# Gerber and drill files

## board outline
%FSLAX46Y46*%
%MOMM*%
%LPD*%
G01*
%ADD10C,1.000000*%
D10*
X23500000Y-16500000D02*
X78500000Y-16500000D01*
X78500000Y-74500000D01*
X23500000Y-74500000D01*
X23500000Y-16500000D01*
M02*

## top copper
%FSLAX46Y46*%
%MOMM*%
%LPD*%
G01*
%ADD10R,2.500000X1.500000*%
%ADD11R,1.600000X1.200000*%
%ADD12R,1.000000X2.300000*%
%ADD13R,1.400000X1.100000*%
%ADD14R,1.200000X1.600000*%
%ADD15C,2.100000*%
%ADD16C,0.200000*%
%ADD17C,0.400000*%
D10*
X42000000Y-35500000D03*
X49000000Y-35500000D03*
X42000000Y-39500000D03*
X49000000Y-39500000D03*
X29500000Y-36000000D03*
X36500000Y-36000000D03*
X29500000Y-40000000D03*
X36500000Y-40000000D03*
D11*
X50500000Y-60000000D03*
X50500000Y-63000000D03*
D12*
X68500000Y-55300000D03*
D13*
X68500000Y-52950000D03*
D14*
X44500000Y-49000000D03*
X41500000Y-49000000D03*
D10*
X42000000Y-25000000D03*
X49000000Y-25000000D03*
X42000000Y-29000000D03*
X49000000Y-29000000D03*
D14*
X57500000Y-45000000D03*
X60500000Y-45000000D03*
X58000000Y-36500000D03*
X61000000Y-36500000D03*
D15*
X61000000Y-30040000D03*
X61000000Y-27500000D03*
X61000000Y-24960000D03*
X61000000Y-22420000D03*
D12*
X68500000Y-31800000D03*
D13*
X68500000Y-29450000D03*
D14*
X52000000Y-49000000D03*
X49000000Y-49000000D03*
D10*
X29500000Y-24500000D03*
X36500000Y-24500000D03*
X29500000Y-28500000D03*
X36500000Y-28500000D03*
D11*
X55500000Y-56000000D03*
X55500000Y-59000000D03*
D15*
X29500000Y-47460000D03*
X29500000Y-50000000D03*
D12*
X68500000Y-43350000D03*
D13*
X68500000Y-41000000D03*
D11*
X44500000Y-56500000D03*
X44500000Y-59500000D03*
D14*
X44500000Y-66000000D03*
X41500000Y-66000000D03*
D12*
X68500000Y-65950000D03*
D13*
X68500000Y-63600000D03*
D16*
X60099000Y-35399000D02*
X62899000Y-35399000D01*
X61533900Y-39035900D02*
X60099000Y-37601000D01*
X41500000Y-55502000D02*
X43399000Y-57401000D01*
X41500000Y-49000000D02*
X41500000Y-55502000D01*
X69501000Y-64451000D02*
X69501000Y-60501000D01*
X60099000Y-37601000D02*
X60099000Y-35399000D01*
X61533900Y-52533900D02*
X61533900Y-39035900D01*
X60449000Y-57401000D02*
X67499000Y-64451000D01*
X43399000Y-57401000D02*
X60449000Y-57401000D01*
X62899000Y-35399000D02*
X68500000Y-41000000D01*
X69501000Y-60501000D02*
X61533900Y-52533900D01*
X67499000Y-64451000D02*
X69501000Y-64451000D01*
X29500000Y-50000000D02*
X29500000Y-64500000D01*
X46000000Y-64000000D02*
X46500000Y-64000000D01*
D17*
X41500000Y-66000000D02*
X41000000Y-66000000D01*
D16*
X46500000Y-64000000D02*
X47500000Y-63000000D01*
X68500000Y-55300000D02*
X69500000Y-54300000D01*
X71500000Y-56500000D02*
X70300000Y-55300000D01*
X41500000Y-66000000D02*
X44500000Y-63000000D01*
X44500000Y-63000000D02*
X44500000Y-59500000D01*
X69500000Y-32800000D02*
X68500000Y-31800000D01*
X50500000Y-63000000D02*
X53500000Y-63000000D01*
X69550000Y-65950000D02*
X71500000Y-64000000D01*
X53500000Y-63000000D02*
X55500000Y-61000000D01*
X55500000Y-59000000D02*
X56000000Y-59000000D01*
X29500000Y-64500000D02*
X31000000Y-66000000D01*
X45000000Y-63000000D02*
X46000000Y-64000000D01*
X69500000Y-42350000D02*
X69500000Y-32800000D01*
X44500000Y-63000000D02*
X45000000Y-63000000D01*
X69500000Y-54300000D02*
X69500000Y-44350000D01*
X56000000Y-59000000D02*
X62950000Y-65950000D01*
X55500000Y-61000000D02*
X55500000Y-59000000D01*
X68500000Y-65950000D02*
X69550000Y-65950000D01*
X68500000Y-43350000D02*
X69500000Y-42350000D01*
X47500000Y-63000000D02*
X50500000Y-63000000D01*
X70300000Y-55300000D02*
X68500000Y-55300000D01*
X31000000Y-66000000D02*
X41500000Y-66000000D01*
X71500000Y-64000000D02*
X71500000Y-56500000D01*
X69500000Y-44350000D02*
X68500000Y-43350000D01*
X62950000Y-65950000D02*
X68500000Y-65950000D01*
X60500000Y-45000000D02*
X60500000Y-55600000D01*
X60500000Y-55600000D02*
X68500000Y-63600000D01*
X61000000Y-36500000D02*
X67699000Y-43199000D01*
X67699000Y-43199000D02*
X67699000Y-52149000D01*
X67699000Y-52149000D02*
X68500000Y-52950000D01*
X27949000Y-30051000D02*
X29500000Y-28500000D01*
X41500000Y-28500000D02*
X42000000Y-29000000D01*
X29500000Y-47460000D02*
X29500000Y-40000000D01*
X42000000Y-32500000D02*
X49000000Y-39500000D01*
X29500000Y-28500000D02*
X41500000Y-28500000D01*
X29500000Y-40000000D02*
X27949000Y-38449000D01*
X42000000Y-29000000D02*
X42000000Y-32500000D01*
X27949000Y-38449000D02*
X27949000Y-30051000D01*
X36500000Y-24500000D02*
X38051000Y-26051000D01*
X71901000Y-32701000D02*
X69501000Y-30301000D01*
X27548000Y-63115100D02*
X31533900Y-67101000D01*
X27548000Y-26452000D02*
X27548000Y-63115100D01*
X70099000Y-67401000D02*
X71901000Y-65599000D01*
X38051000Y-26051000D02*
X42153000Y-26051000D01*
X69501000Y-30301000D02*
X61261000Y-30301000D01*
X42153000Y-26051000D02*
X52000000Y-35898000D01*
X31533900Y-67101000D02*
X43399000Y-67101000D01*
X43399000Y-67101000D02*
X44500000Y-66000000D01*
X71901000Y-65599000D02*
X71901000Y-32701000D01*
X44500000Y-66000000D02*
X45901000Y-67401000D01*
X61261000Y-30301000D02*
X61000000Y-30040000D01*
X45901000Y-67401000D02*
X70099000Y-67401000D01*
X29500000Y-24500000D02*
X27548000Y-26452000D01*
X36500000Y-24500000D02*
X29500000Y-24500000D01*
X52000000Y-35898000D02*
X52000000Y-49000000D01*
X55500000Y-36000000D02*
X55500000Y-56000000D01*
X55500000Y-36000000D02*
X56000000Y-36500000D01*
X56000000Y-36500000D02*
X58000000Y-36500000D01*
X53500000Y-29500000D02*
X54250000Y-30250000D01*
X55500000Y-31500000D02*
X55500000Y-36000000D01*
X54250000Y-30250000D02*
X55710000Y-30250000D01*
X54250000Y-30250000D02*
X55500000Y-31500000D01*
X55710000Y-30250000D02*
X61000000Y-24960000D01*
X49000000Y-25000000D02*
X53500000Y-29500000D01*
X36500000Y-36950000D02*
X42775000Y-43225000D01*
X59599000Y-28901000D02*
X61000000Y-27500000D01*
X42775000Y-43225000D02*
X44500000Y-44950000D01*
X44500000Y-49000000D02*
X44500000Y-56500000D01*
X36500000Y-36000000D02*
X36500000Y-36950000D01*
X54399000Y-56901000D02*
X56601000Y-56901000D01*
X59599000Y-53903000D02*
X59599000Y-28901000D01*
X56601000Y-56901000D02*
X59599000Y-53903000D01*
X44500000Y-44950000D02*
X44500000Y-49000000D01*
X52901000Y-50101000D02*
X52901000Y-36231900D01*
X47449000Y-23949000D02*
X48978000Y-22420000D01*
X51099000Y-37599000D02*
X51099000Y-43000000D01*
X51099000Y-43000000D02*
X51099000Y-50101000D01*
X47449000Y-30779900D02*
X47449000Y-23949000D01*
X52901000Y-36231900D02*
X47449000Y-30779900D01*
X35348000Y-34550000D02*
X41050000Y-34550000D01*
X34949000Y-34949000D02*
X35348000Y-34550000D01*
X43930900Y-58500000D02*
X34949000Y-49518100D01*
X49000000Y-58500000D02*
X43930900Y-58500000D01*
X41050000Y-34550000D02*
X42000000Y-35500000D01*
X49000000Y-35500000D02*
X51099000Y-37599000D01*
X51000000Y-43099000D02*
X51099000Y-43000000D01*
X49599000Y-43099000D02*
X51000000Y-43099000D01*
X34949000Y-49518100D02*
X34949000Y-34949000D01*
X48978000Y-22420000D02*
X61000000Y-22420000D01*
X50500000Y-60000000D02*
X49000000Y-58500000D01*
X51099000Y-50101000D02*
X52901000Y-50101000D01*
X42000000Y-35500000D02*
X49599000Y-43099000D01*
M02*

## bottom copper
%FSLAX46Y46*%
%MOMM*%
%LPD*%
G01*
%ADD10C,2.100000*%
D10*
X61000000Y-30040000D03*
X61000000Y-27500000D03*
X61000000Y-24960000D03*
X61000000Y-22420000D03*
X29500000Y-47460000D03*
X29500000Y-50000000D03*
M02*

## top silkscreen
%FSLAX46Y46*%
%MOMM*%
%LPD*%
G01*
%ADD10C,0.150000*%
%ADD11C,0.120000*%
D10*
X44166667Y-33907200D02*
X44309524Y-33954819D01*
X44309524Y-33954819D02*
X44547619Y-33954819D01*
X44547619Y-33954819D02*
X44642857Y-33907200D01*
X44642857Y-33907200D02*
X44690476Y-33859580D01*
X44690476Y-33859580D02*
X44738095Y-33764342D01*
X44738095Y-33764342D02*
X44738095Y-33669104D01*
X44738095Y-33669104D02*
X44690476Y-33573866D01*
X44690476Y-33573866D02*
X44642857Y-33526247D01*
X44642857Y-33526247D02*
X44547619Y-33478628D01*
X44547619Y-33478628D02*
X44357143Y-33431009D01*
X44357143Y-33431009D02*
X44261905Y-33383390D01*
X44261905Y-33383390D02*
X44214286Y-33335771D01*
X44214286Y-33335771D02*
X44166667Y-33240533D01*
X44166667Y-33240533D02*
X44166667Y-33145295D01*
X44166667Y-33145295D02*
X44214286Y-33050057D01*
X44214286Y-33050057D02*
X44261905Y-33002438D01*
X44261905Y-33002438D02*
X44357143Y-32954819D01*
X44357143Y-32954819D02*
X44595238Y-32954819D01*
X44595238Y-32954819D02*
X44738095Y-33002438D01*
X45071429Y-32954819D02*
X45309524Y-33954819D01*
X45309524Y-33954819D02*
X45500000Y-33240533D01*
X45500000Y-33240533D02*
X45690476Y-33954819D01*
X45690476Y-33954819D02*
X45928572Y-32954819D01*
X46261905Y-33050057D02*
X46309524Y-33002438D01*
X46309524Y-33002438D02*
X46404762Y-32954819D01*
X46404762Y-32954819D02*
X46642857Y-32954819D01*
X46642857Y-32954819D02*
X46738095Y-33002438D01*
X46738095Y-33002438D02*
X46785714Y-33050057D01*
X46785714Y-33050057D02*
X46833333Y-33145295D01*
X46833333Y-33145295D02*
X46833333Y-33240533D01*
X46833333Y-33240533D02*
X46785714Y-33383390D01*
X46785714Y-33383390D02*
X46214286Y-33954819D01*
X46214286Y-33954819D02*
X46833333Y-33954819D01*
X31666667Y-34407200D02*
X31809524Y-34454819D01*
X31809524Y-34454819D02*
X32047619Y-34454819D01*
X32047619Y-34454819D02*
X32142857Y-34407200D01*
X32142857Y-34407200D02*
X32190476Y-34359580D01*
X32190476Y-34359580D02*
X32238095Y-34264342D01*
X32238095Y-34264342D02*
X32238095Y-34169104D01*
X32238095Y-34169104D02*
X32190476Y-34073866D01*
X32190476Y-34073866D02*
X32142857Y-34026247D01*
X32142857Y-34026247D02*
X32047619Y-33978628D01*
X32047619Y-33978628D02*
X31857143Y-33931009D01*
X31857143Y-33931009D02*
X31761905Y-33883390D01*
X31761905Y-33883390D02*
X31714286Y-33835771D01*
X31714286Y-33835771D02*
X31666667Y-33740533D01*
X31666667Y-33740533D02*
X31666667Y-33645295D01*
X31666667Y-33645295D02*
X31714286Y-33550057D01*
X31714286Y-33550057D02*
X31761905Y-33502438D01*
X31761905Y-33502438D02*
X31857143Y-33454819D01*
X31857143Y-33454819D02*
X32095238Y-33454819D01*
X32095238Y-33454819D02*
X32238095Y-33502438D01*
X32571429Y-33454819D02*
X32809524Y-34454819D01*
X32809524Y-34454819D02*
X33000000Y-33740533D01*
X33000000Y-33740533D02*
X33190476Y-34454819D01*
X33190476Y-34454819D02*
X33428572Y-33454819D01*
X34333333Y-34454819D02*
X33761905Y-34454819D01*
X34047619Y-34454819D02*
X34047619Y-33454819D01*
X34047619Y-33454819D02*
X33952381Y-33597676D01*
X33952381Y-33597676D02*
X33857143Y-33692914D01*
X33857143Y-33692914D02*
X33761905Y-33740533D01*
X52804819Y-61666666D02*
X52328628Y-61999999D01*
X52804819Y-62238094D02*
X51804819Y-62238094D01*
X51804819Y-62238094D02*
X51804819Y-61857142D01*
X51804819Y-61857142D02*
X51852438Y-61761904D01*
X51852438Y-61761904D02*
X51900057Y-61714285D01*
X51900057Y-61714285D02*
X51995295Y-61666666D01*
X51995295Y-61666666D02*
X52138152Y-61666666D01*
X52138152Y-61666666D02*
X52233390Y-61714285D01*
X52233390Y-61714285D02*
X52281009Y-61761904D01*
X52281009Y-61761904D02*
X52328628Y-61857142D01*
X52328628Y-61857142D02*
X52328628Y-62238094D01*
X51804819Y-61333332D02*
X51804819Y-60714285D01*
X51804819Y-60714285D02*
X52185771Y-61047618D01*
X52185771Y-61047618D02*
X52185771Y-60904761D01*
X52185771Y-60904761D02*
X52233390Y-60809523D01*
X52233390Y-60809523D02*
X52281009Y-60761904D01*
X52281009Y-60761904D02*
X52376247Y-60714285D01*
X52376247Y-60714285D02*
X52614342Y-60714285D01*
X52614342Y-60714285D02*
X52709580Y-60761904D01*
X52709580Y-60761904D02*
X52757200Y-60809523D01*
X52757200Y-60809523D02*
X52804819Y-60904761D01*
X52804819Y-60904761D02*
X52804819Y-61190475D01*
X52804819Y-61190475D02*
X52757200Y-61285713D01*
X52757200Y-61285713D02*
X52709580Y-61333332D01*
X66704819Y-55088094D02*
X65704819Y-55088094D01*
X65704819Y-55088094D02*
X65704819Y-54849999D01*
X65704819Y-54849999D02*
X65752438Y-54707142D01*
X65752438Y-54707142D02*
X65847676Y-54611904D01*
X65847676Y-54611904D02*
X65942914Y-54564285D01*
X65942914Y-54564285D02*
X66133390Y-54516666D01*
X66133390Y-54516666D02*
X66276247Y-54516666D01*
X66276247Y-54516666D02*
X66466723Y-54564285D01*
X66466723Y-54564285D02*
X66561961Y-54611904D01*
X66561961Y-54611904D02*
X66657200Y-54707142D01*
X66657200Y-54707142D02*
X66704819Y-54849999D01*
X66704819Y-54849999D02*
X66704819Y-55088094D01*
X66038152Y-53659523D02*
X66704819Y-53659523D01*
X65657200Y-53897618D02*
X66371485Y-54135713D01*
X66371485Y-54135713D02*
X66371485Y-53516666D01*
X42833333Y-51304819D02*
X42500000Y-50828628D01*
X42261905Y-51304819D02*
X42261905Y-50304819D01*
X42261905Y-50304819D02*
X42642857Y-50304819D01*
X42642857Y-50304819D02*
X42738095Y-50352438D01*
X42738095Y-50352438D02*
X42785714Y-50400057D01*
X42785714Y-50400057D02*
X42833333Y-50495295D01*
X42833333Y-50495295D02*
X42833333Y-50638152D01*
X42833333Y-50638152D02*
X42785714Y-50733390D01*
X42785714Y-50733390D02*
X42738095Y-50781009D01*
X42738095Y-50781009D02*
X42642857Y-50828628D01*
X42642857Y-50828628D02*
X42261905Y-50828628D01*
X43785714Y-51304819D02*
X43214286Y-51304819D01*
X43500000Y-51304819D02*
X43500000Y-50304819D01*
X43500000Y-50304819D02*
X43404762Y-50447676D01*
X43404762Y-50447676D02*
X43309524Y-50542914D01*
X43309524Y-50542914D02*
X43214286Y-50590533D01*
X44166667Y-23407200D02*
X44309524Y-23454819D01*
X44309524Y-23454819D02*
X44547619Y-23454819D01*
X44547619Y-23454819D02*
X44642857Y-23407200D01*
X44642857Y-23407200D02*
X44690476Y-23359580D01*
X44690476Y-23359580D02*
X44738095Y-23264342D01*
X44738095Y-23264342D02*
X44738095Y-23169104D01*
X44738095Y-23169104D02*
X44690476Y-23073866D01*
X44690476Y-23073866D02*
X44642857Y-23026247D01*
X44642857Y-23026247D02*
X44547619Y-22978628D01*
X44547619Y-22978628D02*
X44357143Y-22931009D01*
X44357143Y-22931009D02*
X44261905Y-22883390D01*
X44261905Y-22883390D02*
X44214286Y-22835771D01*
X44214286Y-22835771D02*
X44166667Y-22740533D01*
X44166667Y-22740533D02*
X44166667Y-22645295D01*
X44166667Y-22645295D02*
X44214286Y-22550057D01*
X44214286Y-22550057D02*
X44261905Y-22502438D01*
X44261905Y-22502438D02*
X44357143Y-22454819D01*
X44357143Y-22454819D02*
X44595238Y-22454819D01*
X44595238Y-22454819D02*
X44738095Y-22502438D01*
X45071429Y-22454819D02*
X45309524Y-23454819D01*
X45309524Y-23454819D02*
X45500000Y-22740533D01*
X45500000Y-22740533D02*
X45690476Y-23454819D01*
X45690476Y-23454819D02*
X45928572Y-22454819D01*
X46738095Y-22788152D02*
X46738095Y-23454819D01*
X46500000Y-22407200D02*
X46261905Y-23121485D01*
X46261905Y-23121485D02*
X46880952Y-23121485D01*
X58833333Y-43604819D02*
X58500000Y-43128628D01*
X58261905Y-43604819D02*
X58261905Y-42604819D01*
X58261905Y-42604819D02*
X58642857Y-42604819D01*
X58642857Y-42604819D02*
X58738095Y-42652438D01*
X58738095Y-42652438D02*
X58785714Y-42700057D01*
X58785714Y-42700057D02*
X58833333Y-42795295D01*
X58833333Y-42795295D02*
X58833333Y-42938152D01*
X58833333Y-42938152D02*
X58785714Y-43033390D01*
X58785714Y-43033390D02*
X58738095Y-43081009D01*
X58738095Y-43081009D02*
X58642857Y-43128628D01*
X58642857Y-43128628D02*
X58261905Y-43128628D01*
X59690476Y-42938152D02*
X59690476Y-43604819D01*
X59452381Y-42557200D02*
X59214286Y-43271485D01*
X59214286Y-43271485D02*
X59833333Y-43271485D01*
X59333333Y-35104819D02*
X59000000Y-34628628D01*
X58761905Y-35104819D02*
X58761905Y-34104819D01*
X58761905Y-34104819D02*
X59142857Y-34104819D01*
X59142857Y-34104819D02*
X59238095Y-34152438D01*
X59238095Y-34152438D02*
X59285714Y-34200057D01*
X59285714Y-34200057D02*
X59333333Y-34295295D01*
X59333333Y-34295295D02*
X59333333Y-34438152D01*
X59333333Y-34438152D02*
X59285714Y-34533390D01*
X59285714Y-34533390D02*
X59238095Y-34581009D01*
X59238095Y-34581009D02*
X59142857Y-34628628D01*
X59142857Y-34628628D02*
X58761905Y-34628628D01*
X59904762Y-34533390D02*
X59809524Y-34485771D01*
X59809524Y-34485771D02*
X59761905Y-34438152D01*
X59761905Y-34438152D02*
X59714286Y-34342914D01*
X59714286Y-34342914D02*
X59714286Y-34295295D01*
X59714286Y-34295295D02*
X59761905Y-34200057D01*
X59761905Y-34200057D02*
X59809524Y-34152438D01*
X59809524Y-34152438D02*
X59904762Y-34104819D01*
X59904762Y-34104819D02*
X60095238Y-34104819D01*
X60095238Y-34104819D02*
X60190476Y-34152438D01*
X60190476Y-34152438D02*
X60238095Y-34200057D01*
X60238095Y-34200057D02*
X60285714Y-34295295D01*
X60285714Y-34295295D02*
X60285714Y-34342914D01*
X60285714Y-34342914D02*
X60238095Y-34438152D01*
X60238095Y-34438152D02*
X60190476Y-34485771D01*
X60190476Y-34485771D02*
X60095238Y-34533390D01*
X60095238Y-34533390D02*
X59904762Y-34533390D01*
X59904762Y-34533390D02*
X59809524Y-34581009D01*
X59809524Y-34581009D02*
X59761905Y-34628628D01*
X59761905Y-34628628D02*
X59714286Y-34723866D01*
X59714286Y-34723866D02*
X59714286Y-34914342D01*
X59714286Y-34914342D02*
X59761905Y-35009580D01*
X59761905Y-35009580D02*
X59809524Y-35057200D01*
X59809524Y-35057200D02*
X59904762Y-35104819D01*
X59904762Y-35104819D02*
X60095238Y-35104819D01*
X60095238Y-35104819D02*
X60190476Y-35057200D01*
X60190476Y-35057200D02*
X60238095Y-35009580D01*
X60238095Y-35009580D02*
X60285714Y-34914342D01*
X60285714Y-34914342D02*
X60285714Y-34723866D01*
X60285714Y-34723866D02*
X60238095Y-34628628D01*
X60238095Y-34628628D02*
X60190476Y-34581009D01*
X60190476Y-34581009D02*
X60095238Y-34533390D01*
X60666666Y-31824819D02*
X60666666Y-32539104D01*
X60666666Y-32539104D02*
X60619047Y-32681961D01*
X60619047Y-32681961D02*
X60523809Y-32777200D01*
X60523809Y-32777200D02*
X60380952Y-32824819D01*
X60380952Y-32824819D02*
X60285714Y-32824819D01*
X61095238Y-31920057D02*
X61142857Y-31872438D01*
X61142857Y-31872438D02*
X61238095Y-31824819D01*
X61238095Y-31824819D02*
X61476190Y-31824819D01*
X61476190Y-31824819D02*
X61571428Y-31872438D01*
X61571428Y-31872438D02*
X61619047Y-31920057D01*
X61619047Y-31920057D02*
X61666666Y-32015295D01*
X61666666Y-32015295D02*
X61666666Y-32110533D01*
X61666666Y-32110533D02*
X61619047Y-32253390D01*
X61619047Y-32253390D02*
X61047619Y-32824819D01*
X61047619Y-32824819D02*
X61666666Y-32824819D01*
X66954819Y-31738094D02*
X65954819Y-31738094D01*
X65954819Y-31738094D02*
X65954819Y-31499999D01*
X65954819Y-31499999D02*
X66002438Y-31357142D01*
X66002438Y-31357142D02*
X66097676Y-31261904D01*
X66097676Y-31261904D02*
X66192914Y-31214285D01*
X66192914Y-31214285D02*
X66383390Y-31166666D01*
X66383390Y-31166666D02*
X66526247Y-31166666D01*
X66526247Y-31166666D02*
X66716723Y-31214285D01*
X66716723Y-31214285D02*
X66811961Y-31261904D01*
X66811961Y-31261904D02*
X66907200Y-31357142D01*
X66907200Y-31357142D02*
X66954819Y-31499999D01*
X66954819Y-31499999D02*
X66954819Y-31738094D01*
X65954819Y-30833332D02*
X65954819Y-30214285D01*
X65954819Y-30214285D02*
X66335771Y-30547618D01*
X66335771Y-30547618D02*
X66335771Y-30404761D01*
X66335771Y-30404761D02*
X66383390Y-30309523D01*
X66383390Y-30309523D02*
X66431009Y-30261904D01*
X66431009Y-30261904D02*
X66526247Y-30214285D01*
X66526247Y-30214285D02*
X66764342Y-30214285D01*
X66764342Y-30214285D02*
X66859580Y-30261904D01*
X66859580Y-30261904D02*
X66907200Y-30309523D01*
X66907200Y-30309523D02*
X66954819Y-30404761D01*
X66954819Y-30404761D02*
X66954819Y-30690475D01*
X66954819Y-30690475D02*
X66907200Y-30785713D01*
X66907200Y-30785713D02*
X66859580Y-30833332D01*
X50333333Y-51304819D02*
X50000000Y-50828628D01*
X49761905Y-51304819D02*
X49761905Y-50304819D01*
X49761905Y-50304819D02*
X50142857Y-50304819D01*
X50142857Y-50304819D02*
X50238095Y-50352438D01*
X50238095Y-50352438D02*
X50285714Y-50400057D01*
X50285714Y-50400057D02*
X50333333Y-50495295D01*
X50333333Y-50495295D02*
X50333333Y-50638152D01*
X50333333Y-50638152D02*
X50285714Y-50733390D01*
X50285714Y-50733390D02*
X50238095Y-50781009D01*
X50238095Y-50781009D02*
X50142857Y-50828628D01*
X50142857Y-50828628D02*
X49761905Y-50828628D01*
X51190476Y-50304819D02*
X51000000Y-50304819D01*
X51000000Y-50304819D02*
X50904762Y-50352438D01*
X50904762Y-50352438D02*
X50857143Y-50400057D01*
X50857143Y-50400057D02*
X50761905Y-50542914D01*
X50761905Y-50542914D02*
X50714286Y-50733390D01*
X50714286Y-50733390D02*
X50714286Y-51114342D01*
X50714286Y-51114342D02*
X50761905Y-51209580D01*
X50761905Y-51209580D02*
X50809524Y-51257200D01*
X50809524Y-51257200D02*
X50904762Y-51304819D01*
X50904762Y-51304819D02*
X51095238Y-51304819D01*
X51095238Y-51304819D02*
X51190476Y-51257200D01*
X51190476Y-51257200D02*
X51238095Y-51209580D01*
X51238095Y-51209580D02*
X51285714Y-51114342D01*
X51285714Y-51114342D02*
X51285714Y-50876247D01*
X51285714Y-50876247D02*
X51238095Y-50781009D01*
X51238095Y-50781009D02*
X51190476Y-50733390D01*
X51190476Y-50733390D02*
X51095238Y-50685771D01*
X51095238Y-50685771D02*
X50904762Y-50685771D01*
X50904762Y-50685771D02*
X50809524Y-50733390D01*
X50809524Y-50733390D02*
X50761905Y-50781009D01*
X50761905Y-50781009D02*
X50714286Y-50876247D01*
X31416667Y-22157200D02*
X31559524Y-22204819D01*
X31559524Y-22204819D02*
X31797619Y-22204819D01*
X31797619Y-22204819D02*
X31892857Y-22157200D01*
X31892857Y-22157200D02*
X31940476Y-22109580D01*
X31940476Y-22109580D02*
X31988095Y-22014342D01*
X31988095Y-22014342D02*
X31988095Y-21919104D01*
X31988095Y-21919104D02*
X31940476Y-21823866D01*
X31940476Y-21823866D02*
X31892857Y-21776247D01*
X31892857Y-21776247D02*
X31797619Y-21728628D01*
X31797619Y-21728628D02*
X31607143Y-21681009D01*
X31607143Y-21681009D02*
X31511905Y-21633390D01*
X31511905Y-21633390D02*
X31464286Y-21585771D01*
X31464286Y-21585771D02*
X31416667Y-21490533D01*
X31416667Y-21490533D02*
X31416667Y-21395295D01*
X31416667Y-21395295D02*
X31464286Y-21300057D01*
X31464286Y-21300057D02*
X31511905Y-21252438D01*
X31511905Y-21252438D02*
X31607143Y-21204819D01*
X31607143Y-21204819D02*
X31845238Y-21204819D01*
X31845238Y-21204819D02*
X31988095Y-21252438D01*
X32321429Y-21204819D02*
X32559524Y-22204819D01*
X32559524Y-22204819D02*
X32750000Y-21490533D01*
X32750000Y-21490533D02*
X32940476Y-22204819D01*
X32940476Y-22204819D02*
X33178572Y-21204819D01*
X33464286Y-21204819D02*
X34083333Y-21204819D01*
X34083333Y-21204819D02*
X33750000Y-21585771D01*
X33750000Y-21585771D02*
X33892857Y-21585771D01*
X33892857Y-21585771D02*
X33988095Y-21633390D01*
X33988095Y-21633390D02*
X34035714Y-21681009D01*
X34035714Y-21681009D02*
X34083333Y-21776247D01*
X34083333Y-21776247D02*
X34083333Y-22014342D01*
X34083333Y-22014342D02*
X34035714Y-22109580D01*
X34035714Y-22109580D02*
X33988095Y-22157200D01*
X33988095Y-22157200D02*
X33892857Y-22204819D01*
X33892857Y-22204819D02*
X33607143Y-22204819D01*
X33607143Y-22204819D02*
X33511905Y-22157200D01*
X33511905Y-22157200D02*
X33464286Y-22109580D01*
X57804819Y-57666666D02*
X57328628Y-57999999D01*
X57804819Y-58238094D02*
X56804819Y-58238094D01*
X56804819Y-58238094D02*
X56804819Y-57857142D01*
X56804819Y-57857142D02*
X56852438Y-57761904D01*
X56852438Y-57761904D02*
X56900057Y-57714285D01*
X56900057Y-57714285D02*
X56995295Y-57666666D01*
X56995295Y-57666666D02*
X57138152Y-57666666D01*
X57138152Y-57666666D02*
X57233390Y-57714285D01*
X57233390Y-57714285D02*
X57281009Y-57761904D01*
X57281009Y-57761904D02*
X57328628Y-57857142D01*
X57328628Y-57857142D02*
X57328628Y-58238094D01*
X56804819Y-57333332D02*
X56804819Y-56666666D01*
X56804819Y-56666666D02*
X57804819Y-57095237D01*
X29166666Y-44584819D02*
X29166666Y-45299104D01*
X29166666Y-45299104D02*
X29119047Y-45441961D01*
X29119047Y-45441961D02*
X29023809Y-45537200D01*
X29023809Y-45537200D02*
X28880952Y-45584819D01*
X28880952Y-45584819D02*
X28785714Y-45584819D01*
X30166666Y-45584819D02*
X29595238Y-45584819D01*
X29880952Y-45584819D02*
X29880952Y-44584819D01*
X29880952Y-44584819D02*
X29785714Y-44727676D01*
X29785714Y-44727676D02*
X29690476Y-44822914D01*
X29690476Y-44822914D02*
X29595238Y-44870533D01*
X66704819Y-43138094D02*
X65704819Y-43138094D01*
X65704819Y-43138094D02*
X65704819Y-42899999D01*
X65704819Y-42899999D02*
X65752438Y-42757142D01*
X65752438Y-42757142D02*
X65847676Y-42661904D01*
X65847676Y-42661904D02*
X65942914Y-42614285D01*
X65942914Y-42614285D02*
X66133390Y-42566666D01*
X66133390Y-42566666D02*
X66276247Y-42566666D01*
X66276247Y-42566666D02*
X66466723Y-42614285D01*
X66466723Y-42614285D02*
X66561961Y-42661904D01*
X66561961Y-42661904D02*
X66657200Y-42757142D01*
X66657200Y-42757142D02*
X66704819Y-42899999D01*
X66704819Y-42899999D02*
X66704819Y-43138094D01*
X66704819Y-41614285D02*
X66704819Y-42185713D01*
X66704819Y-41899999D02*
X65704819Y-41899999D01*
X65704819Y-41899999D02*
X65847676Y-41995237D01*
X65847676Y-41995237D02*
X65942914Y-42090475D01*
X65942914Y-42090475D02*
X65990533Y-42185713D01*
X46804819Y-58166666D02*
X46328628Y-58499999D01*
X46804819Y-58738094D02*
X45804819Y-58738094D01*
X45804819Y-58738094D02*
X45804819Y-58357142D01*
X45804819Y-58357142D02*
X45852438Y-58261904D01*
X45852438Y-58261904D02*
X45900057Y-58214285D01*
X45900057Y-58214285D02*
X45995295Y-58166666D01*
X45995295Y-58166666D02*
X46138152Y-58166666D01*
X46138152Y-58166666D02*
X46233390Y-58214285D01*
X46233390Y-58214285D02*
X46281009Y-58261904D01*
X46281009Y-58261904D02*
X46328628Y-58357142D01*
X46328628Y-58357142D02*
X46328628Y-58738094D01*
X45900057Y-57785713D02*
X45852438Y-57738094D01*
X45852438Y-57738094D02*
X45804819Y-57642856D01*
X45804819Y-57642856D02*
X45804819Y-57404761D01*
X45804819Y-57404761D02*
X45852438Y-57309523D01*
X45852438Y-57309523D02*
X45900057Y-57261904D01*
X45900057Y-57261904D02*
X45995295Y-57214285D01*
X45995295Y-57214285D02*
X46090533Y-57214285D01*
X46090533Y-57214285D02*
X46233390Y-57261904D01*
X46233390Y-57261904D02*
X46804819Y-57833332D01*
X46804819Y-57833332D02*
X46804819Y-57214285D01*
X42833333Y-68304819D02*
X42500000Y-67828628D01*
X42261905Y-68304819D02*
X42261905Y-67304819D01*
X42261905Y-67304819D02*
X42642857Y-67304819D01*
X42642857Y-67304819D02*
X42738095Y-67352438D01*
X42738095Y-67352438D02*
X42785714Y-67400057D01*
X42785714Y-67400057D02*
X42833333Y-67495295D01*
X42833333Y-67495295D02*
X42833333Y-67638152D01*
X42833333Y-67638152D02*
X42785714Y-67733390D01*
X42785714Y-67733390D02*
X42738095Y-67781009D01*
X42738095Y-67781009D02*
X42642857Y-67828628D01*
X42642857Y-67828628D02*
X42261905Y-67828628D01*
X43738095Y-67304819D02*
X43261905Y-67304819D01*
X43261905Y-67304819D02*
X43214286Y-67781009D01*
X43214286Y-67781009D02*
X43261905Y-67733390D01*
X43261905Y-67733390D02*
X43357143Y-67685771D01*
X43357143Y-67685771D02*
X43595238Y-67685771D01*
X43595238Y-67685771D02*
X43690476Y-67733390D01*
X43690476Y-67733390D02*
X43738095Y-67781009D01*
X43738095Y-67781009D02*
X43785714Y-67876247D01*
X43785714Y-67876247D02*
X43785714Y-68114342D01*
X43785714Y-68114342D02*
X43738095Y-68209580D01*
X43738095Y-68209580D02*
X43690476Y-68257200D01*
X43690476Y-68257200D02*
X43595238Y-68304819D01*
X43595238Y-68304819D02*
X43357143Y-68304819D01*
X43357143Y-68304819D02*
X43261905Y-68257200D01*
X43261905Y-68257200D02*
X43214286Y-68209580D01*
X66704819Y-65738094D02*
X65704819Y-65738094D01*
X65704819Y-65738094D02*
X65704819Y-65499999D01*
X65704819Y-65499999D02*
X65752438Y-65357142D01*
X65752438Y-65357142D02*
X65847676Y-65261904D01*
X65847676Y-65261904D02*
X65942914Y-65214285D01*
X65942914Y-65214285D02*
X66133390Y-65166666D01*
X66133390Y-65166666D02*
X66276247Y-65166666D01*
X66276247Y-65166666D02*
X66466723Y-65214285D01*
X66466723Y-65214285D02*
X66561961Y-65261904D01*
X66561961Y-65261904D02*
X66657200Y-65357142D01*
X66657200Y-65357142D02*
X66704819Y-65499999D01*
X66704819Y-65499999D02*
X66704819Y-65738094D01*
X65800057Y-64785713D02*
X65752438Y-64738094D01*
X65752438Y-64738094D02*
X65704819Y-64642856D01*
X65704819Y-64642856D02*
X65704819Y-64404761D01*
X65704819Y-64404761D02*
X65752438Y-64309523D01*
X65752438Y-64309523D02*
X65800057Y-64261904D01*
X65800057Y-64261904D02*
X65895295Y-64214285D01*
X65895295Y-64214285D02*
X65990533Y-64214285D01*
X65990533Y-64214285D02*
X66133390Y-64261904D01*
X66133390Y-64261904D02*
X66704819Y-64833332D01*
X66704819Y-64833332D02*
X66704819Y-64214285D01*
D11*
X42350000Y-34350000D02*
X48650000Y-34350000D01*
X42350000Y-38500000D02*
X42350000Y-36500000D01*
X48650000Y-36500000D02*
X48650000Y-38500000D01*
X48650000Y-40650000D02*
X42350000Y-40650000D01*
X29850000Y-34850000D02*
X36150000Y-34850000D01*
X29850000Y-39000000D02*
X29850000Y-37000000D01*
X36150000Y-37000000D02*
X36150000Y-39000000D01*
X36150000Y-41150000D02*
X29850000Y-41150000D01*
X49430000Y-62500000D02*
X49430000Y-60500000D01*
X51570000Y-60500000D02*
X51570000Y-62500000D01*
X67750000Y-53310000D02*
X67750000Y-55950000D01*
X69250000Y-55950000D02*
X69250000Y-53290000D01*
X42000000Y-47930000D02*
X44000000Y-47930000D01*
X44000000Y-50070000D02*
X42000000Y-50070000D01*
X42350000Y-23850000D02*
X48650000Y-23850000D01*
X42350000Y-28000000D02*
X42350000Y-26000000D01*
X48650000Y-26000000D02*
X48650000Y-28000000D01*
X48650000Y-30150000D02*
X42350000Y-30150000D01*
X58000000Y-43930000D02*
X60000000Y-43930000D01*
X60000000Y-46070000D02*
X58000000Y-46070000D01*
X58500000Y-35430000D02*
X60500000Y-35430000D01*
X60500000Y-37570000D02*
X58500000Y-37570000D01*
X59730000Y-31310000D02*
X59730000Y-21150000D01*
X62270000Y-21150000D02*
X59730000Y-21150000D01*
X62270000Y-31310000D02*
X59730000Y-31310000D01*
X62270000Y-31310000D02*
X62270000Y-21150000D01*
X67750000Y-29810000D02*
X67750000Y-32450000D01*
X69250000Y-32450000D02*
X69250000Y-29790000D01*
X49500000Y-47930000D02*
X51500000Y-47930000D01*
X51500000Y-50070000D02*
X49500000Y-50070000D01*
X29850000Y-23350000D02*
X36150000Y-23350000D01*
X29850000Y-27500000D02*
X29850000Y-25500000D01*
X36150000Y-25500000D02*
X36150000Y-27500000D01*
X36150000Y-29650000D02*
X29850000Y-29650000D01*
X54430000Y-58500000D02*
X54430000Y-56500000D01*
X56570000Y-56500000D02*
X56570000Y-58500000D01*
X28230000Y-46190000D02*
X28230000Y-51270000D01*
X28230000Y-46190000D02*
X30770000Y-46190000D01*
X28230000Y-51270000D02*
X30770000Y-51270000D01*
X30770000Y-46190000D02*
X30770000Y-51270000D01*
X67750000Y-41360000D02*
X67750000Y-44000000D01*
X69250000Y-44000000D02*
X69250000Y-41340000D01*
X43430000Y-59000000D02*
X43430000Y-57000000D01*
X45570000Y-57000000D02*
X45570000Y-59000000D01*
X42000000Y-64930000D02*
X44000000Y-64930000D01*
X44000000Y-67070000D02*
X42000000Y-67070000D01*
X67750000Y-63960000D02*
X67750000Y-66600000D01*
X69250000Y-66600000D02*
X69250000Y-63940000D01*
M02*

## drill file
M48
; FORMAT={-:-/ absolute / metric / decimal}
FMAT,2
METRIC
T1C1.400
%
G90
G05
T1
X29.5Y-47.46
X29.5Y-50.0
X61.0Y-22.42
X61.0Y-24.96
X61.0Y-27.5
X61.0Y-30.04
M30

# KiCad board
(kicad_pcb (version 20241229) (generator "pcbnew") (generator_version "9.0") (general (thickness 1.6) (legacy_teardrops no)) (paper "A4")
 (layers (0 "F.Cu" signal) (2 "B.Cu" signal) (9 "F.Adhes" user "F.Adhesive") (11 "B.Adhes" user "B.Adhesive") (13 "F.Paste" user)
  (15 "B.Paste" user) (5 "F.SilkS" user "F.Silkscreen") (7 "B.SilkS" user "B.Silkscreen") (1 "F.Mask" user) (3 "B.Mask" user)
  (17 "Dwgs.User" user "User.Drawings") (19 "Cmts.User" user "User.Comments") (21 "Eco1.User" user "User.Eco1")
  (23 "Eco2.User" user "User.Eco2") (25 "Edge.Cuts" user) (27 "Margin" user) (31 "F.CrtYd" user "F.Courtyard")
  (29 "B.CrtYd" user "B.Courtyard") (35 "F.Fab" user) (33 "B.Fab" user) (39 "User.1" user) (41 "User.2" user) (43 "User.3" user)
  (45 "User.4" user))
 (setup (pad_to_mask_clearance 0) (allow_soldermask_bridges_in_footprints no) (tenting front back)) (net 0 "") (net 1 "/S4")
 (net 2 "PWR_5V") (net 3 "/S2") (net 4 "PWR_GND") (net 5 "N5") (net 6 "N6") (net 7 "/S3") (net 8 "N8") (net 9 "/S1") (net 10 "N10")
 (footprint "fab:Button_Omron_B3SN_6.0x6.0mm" (layer "F.Cu") (at 45.5 37.5)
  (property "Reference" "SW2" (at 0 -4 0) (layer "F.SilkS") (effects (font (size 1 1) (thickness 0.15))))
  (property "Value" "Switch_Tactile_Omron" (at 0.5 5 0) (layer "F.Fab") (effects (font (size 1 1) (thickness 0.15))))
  (fp_line (start -3.15 -3.15) (end 3.15 -3.15) (stroke (width 0.12) (type solid)) (layer "F.SilkS"))
  (fp_line (start -3.15 1) (end -3.15 -1) (stroke (width 0.12) (type solid)) (layer "F.SilkS"))
  (fp_line (start 3.15 -1) (end 3.15 1) (stroke (width 0.12) (type solid)) (layer "F.SilkS"))
  (fp_line (start 3.15 3.15) (end -3.15 3.15) (stroke (width 0.12) (type solid)) (layer "F.SilkS"))
  (pad "1" smd rect (at -3.5 -2) (size 2.5 1.5) (layers "F.Cu" "F.Mask" "F.Paste") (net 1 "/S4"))
  (pad "1" smd rect (at 3.5 -2) (size 2.5 1.5) (layers "F.Cu" "F.Mask" "F.Paste") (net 1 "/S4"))
  (pad "2" smd rect (at -3.5 2) (size 2.5 1.5) (layers "F.Cu" "F.Mask" "F.Paste") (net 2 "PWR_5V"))
  (pad "2" smd rect (at 3.5 2) (size 2.5 1.5) (layers "F.Cu" "F.Mask" "F.Paste") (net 2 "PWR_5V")))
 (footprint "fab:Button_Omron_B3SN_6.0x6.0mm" (layer "F.Cu") (at 33 38)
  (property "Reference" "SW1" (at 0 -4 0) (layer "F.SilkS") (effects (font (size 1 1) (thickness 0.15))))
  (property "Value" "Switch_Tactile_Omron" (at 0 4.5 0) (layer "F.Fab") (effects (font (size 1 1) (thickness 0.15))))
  (fp_line (start -3.15 -3.15) (end 3.15 -3.15) (stroke (width 0.12) (type solid)) (layer "F.SilkS"))
  (fp_line (start -3.15 1) (end -3.15 -1) (stroke (width 0.12) (type solid)) (layer "F.SilkS"))
  (fp_line (start 3.15 -1) (end 3.15 1) (stroke (width 0.12) (type solid)) (layer "F.SilkS"))
  (fp_line (start 3.15 3.15) (end -3.15 3.15) (stroke (width 0.12) (type solid)) (layer "F.SilkS"))
  (pad "1" smd rect (at -3.5 -2) (size 2.5 1.5) (layers "F.Cu" "F.Mask" "F.Paste") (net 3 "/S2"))
  (pad "1" smd rect (at 3.5 -2) (size 2.5 1.5) (layers "F.Cu" "F.Mask" "F.Paste") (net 3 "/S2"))
  (pad "2" smd rect (at -3.5 2) (size 2.5 1.5) (layers "F.Cu" "F.Mask" "F.Paste") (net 2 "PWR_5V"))
  (pad "2" smd rect (at 3.5 2) (size 2.5 1.5) (layers "F.Cu" "F.Mask" "F.Paste") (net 2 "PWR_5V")))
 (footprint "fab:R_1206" (layer "F.Cu") (at 50.5 61.5 -90)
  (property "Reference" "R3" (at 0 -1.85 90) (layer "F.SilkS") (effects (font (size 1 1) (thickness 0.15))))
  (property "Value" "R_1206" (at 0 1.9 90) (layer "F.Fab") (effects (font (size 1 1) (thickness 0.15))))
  (fp_line (start 1 1.07) (end -1 1.07) (stroke (width 0.12) (type solid)) (layer "F.SilkS"))
  (fp_line (start -1 -1.07) (end 1 -1.07) (stroke (width 0.12) (type solid)) (layer "F.SilkS"))
  (pad "1" smd rect (at -1.5 0 270) (size 1.2 1.6) (layers "F.Cu" "F.Mask" "F.Paste") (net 1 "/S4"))
  (pad "2" smd rect (at 1.5 0 270) (size 1.2 1.6) (layers "F.Cu" "F.Mask" "F.Paste") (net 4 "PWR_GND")))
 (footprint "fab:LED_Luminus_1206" (layer "F.Cu") (at 68.5 54.35 -90)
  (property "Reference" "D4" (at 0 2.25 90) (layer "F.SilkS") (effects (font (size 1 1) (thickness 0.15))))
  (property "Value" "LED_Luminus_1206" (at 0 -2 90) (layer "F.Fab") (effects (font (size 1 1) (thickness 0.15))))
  (fp_line (start -1.04 0.75) (end 1.6 0.75) (stroke (width 0.12) (type solid)) (layer "F.SilkS"))
  (fp_line (start 1.6 -0.75) (end -1.06 -0.75) (stroke (width 0.12) (type solid)) (layer "F.SilkS"))
  (pad "1" smd rect (at 0.95 0 270) (size 2.3 1) (layers "F.Cu" "F.Mask" "F.Paste") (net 4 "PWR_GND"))
  (pad "2" smd rect (at -1.4 0 270) (size 1.1 1.4) (layers "F.Cu" "F.Mask" "F.Paste") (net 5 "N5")))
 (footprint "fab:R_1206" (layer "F.Cu") (at 43 49 180)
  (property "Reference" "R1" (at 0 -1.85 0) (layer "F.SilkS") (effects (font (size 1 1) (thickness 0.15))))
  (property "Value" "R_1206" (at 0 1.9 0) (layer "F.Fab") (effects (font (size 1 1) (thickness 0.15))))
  (fp_line (start 1 1.07) (end -1 1.07) (stroke (width 0.12) (type solid)) (layer "F.SilkS"))
  (fp_line (start -1 -1.07) (end 1 -1.07) (stroke (width 0.12) (type solid)) (layer "F.SilkS"))
  (pad "1" smd rect (at -1.5 0 180) (size 1.2 1.6) (layers "F.Cu" "F.Mask" "F.Paste") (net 3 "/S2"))
  (pad "2" smd rect (at 1.5 0 180) (size 1.2 1.6) (layers "F.Cu" "F.Mask" "F.Paste") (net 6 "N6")))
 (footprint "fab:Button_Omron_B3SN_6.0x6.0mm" (layer "F.Cu") (at 45.5 27)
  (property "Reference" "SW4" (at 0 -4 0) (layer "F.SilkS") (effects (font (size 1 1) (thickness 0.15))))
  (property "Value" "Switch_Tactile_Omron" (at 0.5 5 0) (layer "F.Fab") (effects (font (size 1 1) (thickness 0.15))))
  (fp_line (start -3.15 -3.15) (end 3.15 -3.15) (stroke (width 0.12) (type solid)) (layer "F.SilkS"))
  (fp_line (start -3.15 1) (end -3.15 -1) (stroke (width 0.12) (type solid)) (layer "F.SilkS"))
  (fp_line (start 3.15 -1) (end 3.15 1) (stroke (width 0.12) (type solid)) (layer "F.SilkS"))
  (fp_line (start 3.15 3.15) (end -3.15 3.15) (stroke (width 0.12) (type solid)) (layer "F.SilkS"))
  (pad "1" smd rect (at -3.5 -2) (size 2.5 1.5) (layers "F.Cu" "F.Mask" "F.Paste") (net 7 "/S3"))
  (pad "1" smd rect (at 3.5 -2) (size 2.5 1.5) (layers "F.Cu" "F.Mask" "F.Paste") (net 7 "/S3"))
  (pad "2" smd rect (at -3.5 2) (size 2.5 1.5) (layers "F.Cu" "F.Mask" "F.Paste") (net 2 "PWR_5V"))
  (pad "2" smd rect (at 3.5 2) (size 2.5 1.5) (layers "F.Cu" "F.Mask" "F.Paste") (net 2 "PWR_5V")))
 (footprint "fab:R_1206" (layer "F.Cu") (at 59 45)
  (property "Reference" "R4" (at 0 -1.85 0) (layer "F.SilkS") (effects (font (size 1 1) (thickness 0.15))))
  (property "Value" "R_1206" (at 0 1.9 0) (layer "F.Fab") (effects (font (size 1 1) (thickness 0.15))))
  (fp_line (start -1 -1.07) (end 1 -1.07) (stroke (width 0.12) (type solid)) (layer "F.SilkS"))
  (fp_line (start 1 1.07) (end -1 1.07) (stroke (width 0.12) (type solid)) (layer "F.SilkS"))
  (pad "1" smd rect (at -1.5 0) (size 1.2 1.6) (layers "F.Cu" "F.Mask" "F.Paste") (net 1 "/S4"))
  (pad "2" smd rect (at 1.5 0) (size 1.2 1.6) (layers "F.Cu" "F.Mask" "F.Paste") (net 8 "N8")))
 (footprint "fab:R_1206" (layer "F.Cu") (at 59.5 36.5)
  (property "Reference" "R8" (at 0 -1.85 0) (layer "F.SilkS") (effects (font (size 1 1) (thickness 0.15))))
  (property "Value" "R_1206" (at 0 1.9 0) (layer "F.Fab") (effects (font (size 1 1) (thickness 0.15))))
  (fp_line (start -1 -1.07) (end 1 -1.07) (stroke (width 0.12) (type solid)) (layer "F.SilkS"))
  (fp_line (start 1 1.07) (end -1 1.07) (stroke (width 0.12) (type solid)) (layer "F.SilkS"))
  (pad "1" smd rect (at -1.5 0) (size 1.2 1.6) (layers "F.Cu" "F.Mask" "F.Paste") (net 7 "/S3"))
  (pad "2" smd rect (at 1.5 0) (size 1.2 1.6) (layers "F.Cu" "F.Mask" "F.Paste") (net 5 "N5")))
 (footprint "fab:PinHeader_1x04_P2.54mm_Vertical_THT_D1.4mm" (layer "F.Cu") (at 61 30.04 180)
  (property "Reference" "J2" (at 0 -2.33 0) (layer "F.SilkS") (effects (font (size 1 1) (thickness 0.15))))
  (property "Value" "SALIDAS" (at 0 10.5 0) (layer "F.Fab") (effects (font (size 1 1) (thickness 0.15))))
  (fp_line (start 1.27 -1.27) (end 1.27 8.89) (stroke (width 0.12) (type solid)) (layer "F.SilkS"))
  (fp_line (start -1.27 8.89) (end 1.27 8.89) (stroke (width 0.12) (type solid)) (layer "F.SilkS"))
  (fp_line (start -1.27 -1.27) (end 1.27 -1.27) (stroke (width 0.12) (type solid)) (layer "F.SilkS"))
  (fp_line (start -1.27 -1.27) (end -1.27 8.89) (stroke (width 0.12) (type solid)) (layer "F.SilkS"))
  (pad "1" thru_hole circle (at 0 0 180) (size 2.1 2.1) (drill 1.4) (layers "*.Cu" "*.Mask") (remove_unused_layers no) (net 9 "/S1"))
  (pad "2" thru_hole circle (at 0 2.54 180) (size 2.1 2.1) (drill 1.4) (layers "*.Cu" "*.Mask") (remove_unused_layers no) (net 3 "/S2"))
  (pad "3" thru_hole circle (at 0 5.08 180) (size 2.1 2.1) (drill 1.4) (layers "*.Cu" "*.Mask") (remove_unused_layers no) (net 7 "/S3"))
  (pad "4" thru_hole circle (at 0 7.62 180) (size 2.1 2.1) (drill 1.4) (layers "*.Cu" "*.Mask") (remove_unused_layers no) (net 1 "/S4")))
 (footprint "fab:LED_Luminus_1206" (layer "F.Cu") (at 68.5 30.85 -90)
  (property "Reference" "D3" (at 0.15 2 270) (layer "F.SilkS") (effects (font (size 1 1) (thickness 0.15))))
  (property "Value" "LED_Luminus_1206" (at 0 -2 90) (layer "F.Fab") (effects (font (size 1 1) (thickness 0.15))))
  (fp_line (start -1.04 0.75) (end 1.6 0.75) (stroke (width 0.12) (type solid)) (layer "F.SilkS"))
  (fp_line (start 1.6 -0.75) (end -1.06 -0.75) (stroke (width 0.12) (type solid)) (layer "F.SilkS"))
  (pad "1" smd rect (at 0.95 0 270) (size 2.3 1) (layers "F.Cu" "F.Mask" "F.Paste") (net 4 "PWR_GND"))
  (pad "2" smd rect (at -1.4 0 270) (size 1.1 1.4) (layers "F.Cu" "F.Mask" "F.Paste") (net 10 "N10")))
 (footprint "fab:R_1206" (layer "F.Cu") (at 50.5 49 180)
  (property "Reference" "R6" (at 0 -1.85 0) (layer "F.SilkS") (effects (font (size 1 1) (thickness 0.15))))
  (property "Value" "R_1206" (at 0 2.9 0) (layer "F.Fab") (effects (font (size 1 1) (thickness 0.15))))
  (fp_line (start 1 1.07) (end -1 1.07) (stroke (width 0.12) (type solid)) (layer "F.SilkS"))
  (fp_line (start -1 -1.07) (end 1 -1.07) (stroke (width 0.12) (type solid)) (layer "F.SilkS"))
  (pad "1" smd rect (at -1.5 0 180) (size 1.2 1.6) (layers "F.Cu" "F.Mask" "F.Paste") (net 9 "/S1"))
  (pad "2" smd rect (at 1.5 0 180) (size 1.2 1.6) (layers "F.Cu" "F.Mask" "F.Paste") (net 10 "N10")))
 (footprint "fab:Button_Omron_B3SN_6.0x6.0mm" (layer "F.Cu") (at 33 26.5)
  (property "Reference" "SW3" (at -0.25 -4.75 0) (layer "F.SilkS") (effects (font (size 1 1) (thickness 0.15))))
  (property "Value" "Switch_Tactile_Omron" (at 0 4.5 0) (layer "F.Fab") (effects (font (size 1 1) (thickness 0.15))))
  (fp_line (start -3.15 -3.15) (end 3.15 -3.15) (stroke (width 0.12) (type solid)) (layer "F.SilkS"))
  (fp_line (start -3.15 1) (end -3.15 -1) (stroke (width 0.12) (type solid)) (layer "F.SilkS"))
  (fp_line (start 3.15 -1) (end 3.15 1) (stroke (width 0.12) (type solid)) (layer "F.SilkS"))
  (fp_line (start 3.15 3.15) (end -3.15 3.15) (stroke (width 0.12) (type solid)) (layer "F.SilkS"))
  (pad "1" smd rect (at -3.5 -2) (size 2.5 1.5) (layers "F.Cu" "F.Mask" "F.Paste") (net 9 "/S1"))
  (pad "1" smd rect (at 3.5 -2) (size 2.5 1.5) (layers "F.Cu" "F.Mask" "F.Paste") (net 9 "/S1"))
  (pad "2" smd rect (at -3.5 2) (size 2.5 1.5) (layers "F.Cu" "F.Mask" "F.Paste") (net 2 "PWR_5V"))
  (pad "2" smd rect (at 3.5 2) (size 2.5 1.5) (layers "F.Cu" "F.Mask" "F.Paste") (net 2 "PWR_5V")))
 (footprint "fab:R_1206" (layer "F.Cu") (at 55.5 57.5 -90)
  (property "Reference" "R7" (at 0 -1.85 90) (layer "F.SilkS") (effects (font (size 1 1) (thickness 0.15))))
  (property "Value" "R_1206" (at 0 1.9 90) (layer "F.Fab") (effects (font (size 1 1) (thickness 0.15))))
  (fp_line (start 1 1.07) (end -1 1.07) (stroke (width 0.12) (type solid)) (layer "F.SilkS"))
  (fp_line (start -1 -1.07) (end 1 -1.07) (stroke (width 0.12) (type solid)) (layer "F.SilkS"))
  (pad "1" smd rect (at -1.5 0 270) (size 1.2 1.6) (layers "F.Cu" "F.Mask" "F.Paste") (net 7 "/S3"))
  (pad "2" smd rect (at 1.5 0 270) (size 1.2 1.6) (layers "F.Cu" "F.Mask" "F.Paste") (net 4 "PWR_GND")))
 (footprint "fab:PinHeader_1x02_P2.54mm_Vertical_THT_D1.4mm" (layer "F.Cu") (at 29.5 47.46)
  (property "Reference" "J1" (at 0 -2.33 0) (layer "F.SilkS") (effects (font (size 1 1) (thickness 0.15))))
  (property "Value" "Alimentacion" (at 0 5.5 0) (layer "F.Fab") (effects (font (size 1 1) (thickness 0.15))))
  (fp_line (start -1.27 -1.27) (end -1.27 3.81) (stroke (width 0.12) (type solid)) (layer "F.SilkS"))
  (fp_line (start -1.27 -1.27) (end 1.27 -1.27) (stroke (width 0.12) (type solid)) (layer "F.SilkS"))
  (fp_line (start -1.27 3.81) (end 1.27 3.81) (stroke (width 0.12) (type solid)) (layer "F.SilkS"))
  (fp_line (start 1.27 -1.27) (end 1.27 3.81) (stroke (width 0.12) (type solid)) (layer "F.SilkS"))
  (pad "1" thru_hole circle (at 0 0) (size 2.1 2.1) (drill 1.4) (layers "*.Cu" "*.Mask") (remove_unused_layers no) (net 2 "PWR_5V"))
  (pad "2" thru_hole circle (at 0 2.54) (size 2.1 2.1) (drill 1.4) (layers "*.Cu" "*.Mask") (remove_unused_layers no) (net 4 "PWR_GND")))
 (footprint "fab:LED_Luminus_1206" (layer "F.Cu") (at 68.5 42.4 -90)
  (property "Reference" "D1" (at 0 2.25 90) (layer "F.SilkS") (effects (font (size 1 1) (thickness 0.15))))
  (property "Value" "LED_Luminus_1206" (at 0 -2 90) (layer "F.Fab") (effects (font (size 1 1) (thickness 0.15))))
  (fp_line (start -1.04 0.75) (end 1.6 0.75) (stroke (width 0.12) (type solid)) (layer "F.SilkS"))
  (fp_line (start 1.6 -0.75) (end -1.06 -0.75) (stroke (width 0.12) (type solid)) (layer "F.SilkS"))
  (pad "1" smd rect (at 0.95 0 270) (size 2.3 1) (layers "F.Cu" "F.Mask" "F.Paste") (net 4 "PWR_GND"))
  (pad "2" smd rect (at -1.4 0 270) (size 1.1 1.4) (layers "F.Cu" "F.Mask" "F.Paste") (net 6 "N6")))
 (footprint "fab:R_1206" (layer "F.Cu") (at 44.5 58 -90)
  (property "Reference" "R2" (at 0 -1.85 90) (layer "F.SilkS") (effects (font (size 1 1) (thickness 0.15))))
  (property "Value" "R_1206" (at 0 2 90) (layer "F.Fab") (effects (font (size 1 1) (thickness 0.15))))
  (fp_line (start 1 1.07) (end -1 1.07) (stroke (width 0.12) (type solid)) (layer "F.SilkS"))
  (fp_line (start -1 -1.07) (end 1 -1.07) (stroke (width 0.12) (type solid)) (layer "F.SilkS"))
  (pad "1" smd rect (at -1.5 0 270) (size 1.2 1.6) (layers "F.Cu" "F.Mask" "F.Paste") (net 3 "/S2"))
  (pad "2" smd rect (at 1.5 0 270) (size 1.2 1.6) (layers "F.Cu" "F.Mask" "F.Paste") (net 4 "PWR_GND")))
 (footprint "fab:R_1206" (layer "F.Cu") (at 43 66 180)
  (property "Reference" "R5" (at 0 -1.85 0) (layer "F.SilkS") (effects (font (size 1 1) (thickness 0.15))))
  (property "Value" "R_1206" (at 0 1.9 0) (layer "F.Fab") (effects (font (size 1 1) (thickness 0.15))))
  (fp_line (start 1 1.07) (end -1 1.07) (stroke (width 0.12) (type solid)) (layer "F.SilkS"))
  (fp_line (start -1 -1.07) (end 1 -1.07) (stroke (width 0.12) (type solid)) (layer "F.SilkS"))
  (pad "1" smd rect (at -1.5 0 180) (size 1.2 1.6) (layers "F.Cu" "F.Mask" "F.Paste") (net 9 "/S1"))
  (pad "2" smd rect (at 1.5 0 180) (size 1.2 1.6) (layers "F.Cu" "F.Mask" "F.Paste") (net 4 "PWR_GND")))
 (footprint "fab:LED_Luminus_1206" (layer "F.Cu") (at 68.5 65 -90)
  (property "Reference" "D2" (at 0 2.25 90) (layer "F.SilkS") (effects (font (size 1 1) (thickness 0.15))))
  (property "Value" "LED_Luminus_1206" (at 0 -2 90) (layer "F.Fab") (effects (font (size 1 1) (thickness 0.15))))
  (fp_line (start -1.04 0.75) (end 1.6 0.75) (stroke (width 0.12) (type solid)) (layer "F.SilkS"))
  (fp_line (start 1.6 -0.75) (end -1.06 -0.75) (stroke (width 0.12) (type solid)) (layer "F.SilkS"))
  (pad "1" smd rect (at 0.95 0 270) (size 2.3 1) (layers "F.Cu" "F.Mask" "F.Paste") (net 4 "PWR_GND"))
  (pad "2" smd rect (at -1.4 0 270) (size 1.1 1.4) (layers "F.Cu" "F.Mask" "F.Paste") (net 8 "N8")))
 (gr_rect (start 23.5 16.5) (end 78.5 74.5) (stroke (width 1) (type solid)) (fill no) (layer "Edge.Cuts"))
 (segment (start 60.099 35.399) (end 62.899 35.399) (width 0.2) (layer "F.Cu") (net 6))
 (segment (start 61.5339 39.0359) (end 60.099 37.601) (width 0.2) (layer "F.Cu") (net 6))
 (segment (start 41.5 55.502) (end 43.399 57.401) (width 0.2) (layer "F.Cu") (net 6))
 (segment (start 41.5 49) (end 41.5 55.502) (width 0.2) (layer "F.Cu") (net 6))
 (segment (start 69.501 64.451) (end 69.501 60.501) (width 0.2) (layer "F.Cu") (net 6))
 (segment (start 60.099 37.601) (end 60.099 35.399) (width 0.2) (layer "F.Cu") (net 6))
 (segment (start 61.5339 52.5339) (end 61.5339 39.0359) (width 0.2) (layer "F.Cu") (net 6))
 (segment (start 60.449 57.401) (end 67.499 64.451) (width 0.2) (layer "F.Cu") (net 6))
 (segment (start 43.399 57.401) (end 60.449 57.401) (width 0.2) (layer "F.Cu") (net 6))
 (segment (start 62.899 35.399) (end 68.5 41) (width 0.2) (layer "F.Cu") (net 6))
 (segment (start 69.501 60.501) (end 61.5339 52.5339) (width 0.2) (layer "F.Cu") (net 6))
 (segment (start 67.499 64.451) (end 69.501 64.451) (width 0.2) (layer "F.Cu") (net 6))
 (segment (start 29.5 50) (end 29.5 64.5) (width 0.2) (layer "F.Cu") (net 4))
 (segment (start 46 64) (end 46.5 64) (width 0.2) (layer "F.Cu") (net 4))
 (segment (start 41.5 66) (end 41 66) (width 0.4) (layer "F.Cu") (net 4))
 (segment (start 46.5 64) (end 47.5 63) (width 0.2) (layer "F.Cu") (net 4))
 (segment (start 68.5 55.3) (end 69.5 54.3) (width 0.2) (layer "F.Cu") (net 4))
 (segment (start 71.5 56.5) (end 70.3 55.3) (width 0.2) (layer "F.Cu") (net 4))
 (segment (start 41.5 66) (end 44.5 63) (width 0.2) (layer "F.Cu") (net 4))
 (segment (start 44.5 63) (end 44.5 59.5) (width 0.2) (layer "F.Cu") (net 4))
 (segment (start 69.5 32.8) (end 68.5 31.8) (width 0.2) (layer "F.Cu") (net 4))
 (segment (start 50.5 63) (end 53.5 63) (width 0.2) (layer "F.Cu") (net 4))
 (segment (start 69.55 65.95) (end 71.5 64) (width 0.2) (layer "F.Cu") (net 4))
 (segment (start 53.5 63) (end 55.5 61) (width 0.2) (layer "F.Cu") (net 4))
 (segment (start 55.5 59) (end 56 59) (width 0.2) (layer "F.Cu") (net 4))
 (segment (start 29.5 64.5) (end 31 66) (width 0.2) (layer "F.Cu") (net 4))
 (segment (start 45 63) (end 46 64) (width 0.2) (layer "F.Cu") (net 4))
 (segment (start 69.5 42.35) (end 69.5 32.8) (width 0.2) (layer "F.Cu") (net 4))
 (segment (start 44.5 63) (end 45 63) (width 0.2) (layer "F.Cu") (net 4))
 (segment (start 69.5 54.3) (end 69.5 44.35) (width 0.2) (layer "F.Cu") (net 4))
 (segment (start 56 59) (end 62.95 65.95) (width 0.2) (layer "F.Cu") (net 4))
 (segment (start 55.5 61) (end 55.5 59) (width 0.2) (layer "F.Cu") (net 4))
 (segment (start 68.5 65.95) (end 69.55 65.95) (width 0.2) (layer "F.Cu") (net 4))
 (segment (start 68.5 43.35) (end 69.5 42.35) (width 0.2) (layer "F.Cu") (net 4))
 (segment (start 47.5 63) (end 50.5 63) (width 0.2) (layer "F.Cu") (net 4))
 (segment (start 70.3 55.3) (end 68.5 55.3) (width 0.2) (layer "F.Cu") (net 4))
 (segment (start 31 66) (end 41.5 66) (width 0.2) (layer "F.Cu") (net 4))
 (segment (start 71.5 64) (end 71.5 56.5) (width 0.2) (layer "F.Cu") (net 4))
 (segment (start 69.5 44.35) (end 68.5 43.35) (width 0.2) (layer "F.Cu") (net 4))
 (segment (start 62.95 65.95) (end 68.5 65.95) (width 0.2) (layer "F.Cu") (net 4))
 (segment (start 60.5 45) (end 60.5 55.6) (width 0.2) (layer "F.Cu") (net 8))
 (segment (start 60.5 55.6) (end 68.5 63.6) (width 0.2) (layer "F.Cu") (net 8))
 (segment (start 61 36.5) (end 67.699 43.199) (width 0.2) (layer "F.Cu") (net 5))
 (segment (start 67.699 43.199) (end 67.699 52.149) (width 0.2) (layer "F.Cu") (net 5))
 (segment (start 67.699 52.149) (end 68.5 52.95) (width 0.2) (layer "F.Cu") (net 5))
 (segment (start 27.949 30.051) (end 29.5 28.5) (width 0.2) (layer "F.Cu") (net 2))
 (segment (start 41.5 28.5) (end 42 29) (width 0.2) (layer "F.Cu") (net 2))
 (segment (start 29.5 47.46) (end 29.5 40) (width 0.2) (layer "F.Cu") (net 2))
 (segment (start 42 32.5) (end 49 39.5) (width 0.2) (layer "F.Cu") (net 2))
 (segment (start 29.5 28.5) (end 41.5 28.5) (width 0.2) (layer "F.Cu") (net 2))
 (segment (start 29.5 40) (end 27.949 38.449) (width 0.2) (layer "F.Cu") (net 2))
 (segment (start 42 29) (end 42 32.5) (width 0.2) (layer "F.Cu") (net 2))
 (segment (start 27.949 38.449) (end 27.949 30.051) (width 0.2) (layer "F.Cu") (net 2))
 (segment (start 36.5 24.5) (end 38.051 26.051) (width 0.2) (layer "F.Cu") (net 9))
 (segment (start 71.901 32.701) (end 69.501 30.301) (width 0.2) (layer "F.Cu") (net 9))
 (segment (start 27.548 63.1151) (end 31.5339 67.101) (width 0.2) (layer "F.Cu") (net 9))
 (segment (start 27.548 26.452) (end 27.548 63.1151) (width 0.2) (layer "F.Cu") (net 9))
 (segment (start 70.099 67.401) (end 71.901 65.599) (width 0.2) (layer "F.Cu") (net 9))
 (segment (start 38.051 26.051) (end 42.153 26.051) (width 0.2) (layer "F.Cu") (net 9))
 (segment (start 69.501 30.301) (end 61.261 30.301) (width 0.2) (layer "F.Cu") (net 9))
 (segment (start 42.153 26.051) (end 52 35.898) (width 0.2) (layer "F.Cu") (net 9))
 (segment (start 31.5339 67.101) (end 43.399 67.101) (width 0.2) (layer "F.Cu") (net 9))
 (segment (start 43.399 67.101) (end 44.5 66) (width 0.2) (layer "F.Cu") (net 9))
 (segment (start 71.901 65.599) (end 71.901 32.701) (width 0.2) (layer "F.Cu") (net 9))
 (segment (start 44.5 66) (end 45.901 67.401) (width 0.2) (layer "F.Cu") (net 9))
 (segment (start 61.261 30.301) (end 61 30.04) (width 0.2) (layer "F.Cu") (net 9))
 (segment (start 45.901 67.401) (end 70.099 67.401) (width 0.2) (layer "F.Cu") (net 9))
 (segment (start 29.5 24.5) (end 27.548 26.452) (width 0.2) (layer "F.Cu") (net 9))
 (segment (start 36.5 24.5) (end 29.5 24.5) (width 0.2) (layer "F.Cu") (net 9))
 (segment (start 52 35.898) (end 52 49) (width 0.2) (layer "F.Cu") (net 9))
 (segment (start 55.5 36) (end 55.5 56) (width 0.2) (layer "F.Cu") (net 7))
 (segment (start 55.5 36) (end 56 36.5) (width 0.2) (layer "F.Cu") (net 7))
 (segment (start 56 36.5) (end 58 36.5) (width 0.2) (layer "F.Cu") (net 7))
 (segment (start 53.5 29.5) (end 54.25 30.25) (width 0.2) (layer "F.Cu") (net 7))
 (segment (start 55.5 31.5) (end 55.5 36) (width 0.2) (layer "F.Cu") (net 7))
 (segment (start 54.25 30.25) (end 55.71 30.25) (width 0.2) (layer "F.Cu") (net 7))
 (segment (start 54.25 30.25) (end 55.5 31.5) (width 0.2) (layer "F.Cu") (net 7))
 (segment (start 55.71 30.25) (end 61 24.96) (width 0.2) (layer "F.Cu") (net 7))
 (segment (start 49 25) (end 53.5 29.5) (width 0.2) (layer "F.Cu") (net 7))
 (segment (start 36.5 36.95) (end 42.775 43.225) (width 0.2) (layer "F.Cu") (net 3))
 (segment (start 59.599 28.901) (end 61 27.5) (width 0.2) (layer "F.Cu") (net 3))
 (segment (start 42.775 43.225) (end 44.5 44.95) (width 0.2) (layer "F.Cu") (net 3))
 (segment (start 44.5 49) (end 44.5 56.5) (width 0.2) (layer "F.Cu") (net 3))
 (segment (start 36.5 36) (end 36.5 36.95) (width 0.2) (layer "F.Cu") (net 3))
 (segment (start 54.399 56.901) (end 56.601 56.901) (width 0.2) (layer "F.Cu") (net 3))
 (segment (start 59.599 53.903) (end 59.599 28.901) (width 0.2) (layer "F.Cu") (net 3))
 (segment (start 56.601 56.901) (end 59.599 53.903) (width 0.2) (layer "F.Cu") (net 3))
 (segment (start 44.5 44.95) (end 44.5 49) (width 0.2) (layer "F.Cu") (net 3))
 (segment (start 52.901 50.101) (end 52.901 36.2319) (width 0.2) (layer "F.Cu") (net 1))
 (segment (start 47.449 23.949) (end 48.978 22.42) (width 0.2) (layer "F.Cu") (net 1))
 (segment (start 51.099 37.599) (end 51.099 43) (width 0.2) (layer "F.Cu") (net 1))
 (segment (start 51.099 43) (end 51.099 50.101) (width 0.2) (layer "F.Cu") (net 1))
 (segment (start 47.449 30.7799) (end 47.449 23.949) (width 0.2) (layer "F.Cu") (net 1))
 (segment (start 52.901 36.2319) (end 47.449 30.7799) (width 0.2) (layer "F.Cu") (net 1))
 (segment (start 35.348 34.55) (end 41.05 34.55) (width 0.2) (layer "F.Cu") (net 1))
 (segment (start 34.949 34.949) (end 35.348 34.55) (width 0.2) (layer "F.Cu") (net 1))
 (segment (start 43.9309 58.5) (end 34.949 49.5181) (width 0.2) (layer "F.Cu") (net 1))
 (segment (start 49 58.5) (end 43.9309 58.5) (width 0.2) (layer "F.Cu") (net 1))
 (segment (start 41.05 34.55) (end 42 35.5) (width 0.2) (layer "F.Cu") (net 1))
 (segment (start 49 35.5) (end 51.099 37.599) (width 0.2) (layer "F.Cu") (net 1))
 (segment (start 51 43.099) (end 51.099 43) (width 0.2) (layer "F.Cu") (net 1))
 (segment (start 49.599 43.099) (end 51 43.099) (width 0.2) (layer "F.Cu") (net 1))
 (segment (start 34.949 49.5181) (end 34.949 34.949) (width 0.2) (layer "F.Cu") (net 1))
 (segment (start 48.978 22.42) (end 61 22.42) (width 0.2) (layer "F.Cu") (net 1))
 (segment (start 50.5 60) (end 49 58.5) (width 0.2) (layer "F.Cu") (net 1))
 (segment (start 51.099 50.101) (end 52.901 50.101) (width 0.2) (layer "F.Cu") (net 1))
 (segment (start 42 35.5) (end 49.599 43.099) (width 0.2) (layer "F.Cu") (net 1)))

